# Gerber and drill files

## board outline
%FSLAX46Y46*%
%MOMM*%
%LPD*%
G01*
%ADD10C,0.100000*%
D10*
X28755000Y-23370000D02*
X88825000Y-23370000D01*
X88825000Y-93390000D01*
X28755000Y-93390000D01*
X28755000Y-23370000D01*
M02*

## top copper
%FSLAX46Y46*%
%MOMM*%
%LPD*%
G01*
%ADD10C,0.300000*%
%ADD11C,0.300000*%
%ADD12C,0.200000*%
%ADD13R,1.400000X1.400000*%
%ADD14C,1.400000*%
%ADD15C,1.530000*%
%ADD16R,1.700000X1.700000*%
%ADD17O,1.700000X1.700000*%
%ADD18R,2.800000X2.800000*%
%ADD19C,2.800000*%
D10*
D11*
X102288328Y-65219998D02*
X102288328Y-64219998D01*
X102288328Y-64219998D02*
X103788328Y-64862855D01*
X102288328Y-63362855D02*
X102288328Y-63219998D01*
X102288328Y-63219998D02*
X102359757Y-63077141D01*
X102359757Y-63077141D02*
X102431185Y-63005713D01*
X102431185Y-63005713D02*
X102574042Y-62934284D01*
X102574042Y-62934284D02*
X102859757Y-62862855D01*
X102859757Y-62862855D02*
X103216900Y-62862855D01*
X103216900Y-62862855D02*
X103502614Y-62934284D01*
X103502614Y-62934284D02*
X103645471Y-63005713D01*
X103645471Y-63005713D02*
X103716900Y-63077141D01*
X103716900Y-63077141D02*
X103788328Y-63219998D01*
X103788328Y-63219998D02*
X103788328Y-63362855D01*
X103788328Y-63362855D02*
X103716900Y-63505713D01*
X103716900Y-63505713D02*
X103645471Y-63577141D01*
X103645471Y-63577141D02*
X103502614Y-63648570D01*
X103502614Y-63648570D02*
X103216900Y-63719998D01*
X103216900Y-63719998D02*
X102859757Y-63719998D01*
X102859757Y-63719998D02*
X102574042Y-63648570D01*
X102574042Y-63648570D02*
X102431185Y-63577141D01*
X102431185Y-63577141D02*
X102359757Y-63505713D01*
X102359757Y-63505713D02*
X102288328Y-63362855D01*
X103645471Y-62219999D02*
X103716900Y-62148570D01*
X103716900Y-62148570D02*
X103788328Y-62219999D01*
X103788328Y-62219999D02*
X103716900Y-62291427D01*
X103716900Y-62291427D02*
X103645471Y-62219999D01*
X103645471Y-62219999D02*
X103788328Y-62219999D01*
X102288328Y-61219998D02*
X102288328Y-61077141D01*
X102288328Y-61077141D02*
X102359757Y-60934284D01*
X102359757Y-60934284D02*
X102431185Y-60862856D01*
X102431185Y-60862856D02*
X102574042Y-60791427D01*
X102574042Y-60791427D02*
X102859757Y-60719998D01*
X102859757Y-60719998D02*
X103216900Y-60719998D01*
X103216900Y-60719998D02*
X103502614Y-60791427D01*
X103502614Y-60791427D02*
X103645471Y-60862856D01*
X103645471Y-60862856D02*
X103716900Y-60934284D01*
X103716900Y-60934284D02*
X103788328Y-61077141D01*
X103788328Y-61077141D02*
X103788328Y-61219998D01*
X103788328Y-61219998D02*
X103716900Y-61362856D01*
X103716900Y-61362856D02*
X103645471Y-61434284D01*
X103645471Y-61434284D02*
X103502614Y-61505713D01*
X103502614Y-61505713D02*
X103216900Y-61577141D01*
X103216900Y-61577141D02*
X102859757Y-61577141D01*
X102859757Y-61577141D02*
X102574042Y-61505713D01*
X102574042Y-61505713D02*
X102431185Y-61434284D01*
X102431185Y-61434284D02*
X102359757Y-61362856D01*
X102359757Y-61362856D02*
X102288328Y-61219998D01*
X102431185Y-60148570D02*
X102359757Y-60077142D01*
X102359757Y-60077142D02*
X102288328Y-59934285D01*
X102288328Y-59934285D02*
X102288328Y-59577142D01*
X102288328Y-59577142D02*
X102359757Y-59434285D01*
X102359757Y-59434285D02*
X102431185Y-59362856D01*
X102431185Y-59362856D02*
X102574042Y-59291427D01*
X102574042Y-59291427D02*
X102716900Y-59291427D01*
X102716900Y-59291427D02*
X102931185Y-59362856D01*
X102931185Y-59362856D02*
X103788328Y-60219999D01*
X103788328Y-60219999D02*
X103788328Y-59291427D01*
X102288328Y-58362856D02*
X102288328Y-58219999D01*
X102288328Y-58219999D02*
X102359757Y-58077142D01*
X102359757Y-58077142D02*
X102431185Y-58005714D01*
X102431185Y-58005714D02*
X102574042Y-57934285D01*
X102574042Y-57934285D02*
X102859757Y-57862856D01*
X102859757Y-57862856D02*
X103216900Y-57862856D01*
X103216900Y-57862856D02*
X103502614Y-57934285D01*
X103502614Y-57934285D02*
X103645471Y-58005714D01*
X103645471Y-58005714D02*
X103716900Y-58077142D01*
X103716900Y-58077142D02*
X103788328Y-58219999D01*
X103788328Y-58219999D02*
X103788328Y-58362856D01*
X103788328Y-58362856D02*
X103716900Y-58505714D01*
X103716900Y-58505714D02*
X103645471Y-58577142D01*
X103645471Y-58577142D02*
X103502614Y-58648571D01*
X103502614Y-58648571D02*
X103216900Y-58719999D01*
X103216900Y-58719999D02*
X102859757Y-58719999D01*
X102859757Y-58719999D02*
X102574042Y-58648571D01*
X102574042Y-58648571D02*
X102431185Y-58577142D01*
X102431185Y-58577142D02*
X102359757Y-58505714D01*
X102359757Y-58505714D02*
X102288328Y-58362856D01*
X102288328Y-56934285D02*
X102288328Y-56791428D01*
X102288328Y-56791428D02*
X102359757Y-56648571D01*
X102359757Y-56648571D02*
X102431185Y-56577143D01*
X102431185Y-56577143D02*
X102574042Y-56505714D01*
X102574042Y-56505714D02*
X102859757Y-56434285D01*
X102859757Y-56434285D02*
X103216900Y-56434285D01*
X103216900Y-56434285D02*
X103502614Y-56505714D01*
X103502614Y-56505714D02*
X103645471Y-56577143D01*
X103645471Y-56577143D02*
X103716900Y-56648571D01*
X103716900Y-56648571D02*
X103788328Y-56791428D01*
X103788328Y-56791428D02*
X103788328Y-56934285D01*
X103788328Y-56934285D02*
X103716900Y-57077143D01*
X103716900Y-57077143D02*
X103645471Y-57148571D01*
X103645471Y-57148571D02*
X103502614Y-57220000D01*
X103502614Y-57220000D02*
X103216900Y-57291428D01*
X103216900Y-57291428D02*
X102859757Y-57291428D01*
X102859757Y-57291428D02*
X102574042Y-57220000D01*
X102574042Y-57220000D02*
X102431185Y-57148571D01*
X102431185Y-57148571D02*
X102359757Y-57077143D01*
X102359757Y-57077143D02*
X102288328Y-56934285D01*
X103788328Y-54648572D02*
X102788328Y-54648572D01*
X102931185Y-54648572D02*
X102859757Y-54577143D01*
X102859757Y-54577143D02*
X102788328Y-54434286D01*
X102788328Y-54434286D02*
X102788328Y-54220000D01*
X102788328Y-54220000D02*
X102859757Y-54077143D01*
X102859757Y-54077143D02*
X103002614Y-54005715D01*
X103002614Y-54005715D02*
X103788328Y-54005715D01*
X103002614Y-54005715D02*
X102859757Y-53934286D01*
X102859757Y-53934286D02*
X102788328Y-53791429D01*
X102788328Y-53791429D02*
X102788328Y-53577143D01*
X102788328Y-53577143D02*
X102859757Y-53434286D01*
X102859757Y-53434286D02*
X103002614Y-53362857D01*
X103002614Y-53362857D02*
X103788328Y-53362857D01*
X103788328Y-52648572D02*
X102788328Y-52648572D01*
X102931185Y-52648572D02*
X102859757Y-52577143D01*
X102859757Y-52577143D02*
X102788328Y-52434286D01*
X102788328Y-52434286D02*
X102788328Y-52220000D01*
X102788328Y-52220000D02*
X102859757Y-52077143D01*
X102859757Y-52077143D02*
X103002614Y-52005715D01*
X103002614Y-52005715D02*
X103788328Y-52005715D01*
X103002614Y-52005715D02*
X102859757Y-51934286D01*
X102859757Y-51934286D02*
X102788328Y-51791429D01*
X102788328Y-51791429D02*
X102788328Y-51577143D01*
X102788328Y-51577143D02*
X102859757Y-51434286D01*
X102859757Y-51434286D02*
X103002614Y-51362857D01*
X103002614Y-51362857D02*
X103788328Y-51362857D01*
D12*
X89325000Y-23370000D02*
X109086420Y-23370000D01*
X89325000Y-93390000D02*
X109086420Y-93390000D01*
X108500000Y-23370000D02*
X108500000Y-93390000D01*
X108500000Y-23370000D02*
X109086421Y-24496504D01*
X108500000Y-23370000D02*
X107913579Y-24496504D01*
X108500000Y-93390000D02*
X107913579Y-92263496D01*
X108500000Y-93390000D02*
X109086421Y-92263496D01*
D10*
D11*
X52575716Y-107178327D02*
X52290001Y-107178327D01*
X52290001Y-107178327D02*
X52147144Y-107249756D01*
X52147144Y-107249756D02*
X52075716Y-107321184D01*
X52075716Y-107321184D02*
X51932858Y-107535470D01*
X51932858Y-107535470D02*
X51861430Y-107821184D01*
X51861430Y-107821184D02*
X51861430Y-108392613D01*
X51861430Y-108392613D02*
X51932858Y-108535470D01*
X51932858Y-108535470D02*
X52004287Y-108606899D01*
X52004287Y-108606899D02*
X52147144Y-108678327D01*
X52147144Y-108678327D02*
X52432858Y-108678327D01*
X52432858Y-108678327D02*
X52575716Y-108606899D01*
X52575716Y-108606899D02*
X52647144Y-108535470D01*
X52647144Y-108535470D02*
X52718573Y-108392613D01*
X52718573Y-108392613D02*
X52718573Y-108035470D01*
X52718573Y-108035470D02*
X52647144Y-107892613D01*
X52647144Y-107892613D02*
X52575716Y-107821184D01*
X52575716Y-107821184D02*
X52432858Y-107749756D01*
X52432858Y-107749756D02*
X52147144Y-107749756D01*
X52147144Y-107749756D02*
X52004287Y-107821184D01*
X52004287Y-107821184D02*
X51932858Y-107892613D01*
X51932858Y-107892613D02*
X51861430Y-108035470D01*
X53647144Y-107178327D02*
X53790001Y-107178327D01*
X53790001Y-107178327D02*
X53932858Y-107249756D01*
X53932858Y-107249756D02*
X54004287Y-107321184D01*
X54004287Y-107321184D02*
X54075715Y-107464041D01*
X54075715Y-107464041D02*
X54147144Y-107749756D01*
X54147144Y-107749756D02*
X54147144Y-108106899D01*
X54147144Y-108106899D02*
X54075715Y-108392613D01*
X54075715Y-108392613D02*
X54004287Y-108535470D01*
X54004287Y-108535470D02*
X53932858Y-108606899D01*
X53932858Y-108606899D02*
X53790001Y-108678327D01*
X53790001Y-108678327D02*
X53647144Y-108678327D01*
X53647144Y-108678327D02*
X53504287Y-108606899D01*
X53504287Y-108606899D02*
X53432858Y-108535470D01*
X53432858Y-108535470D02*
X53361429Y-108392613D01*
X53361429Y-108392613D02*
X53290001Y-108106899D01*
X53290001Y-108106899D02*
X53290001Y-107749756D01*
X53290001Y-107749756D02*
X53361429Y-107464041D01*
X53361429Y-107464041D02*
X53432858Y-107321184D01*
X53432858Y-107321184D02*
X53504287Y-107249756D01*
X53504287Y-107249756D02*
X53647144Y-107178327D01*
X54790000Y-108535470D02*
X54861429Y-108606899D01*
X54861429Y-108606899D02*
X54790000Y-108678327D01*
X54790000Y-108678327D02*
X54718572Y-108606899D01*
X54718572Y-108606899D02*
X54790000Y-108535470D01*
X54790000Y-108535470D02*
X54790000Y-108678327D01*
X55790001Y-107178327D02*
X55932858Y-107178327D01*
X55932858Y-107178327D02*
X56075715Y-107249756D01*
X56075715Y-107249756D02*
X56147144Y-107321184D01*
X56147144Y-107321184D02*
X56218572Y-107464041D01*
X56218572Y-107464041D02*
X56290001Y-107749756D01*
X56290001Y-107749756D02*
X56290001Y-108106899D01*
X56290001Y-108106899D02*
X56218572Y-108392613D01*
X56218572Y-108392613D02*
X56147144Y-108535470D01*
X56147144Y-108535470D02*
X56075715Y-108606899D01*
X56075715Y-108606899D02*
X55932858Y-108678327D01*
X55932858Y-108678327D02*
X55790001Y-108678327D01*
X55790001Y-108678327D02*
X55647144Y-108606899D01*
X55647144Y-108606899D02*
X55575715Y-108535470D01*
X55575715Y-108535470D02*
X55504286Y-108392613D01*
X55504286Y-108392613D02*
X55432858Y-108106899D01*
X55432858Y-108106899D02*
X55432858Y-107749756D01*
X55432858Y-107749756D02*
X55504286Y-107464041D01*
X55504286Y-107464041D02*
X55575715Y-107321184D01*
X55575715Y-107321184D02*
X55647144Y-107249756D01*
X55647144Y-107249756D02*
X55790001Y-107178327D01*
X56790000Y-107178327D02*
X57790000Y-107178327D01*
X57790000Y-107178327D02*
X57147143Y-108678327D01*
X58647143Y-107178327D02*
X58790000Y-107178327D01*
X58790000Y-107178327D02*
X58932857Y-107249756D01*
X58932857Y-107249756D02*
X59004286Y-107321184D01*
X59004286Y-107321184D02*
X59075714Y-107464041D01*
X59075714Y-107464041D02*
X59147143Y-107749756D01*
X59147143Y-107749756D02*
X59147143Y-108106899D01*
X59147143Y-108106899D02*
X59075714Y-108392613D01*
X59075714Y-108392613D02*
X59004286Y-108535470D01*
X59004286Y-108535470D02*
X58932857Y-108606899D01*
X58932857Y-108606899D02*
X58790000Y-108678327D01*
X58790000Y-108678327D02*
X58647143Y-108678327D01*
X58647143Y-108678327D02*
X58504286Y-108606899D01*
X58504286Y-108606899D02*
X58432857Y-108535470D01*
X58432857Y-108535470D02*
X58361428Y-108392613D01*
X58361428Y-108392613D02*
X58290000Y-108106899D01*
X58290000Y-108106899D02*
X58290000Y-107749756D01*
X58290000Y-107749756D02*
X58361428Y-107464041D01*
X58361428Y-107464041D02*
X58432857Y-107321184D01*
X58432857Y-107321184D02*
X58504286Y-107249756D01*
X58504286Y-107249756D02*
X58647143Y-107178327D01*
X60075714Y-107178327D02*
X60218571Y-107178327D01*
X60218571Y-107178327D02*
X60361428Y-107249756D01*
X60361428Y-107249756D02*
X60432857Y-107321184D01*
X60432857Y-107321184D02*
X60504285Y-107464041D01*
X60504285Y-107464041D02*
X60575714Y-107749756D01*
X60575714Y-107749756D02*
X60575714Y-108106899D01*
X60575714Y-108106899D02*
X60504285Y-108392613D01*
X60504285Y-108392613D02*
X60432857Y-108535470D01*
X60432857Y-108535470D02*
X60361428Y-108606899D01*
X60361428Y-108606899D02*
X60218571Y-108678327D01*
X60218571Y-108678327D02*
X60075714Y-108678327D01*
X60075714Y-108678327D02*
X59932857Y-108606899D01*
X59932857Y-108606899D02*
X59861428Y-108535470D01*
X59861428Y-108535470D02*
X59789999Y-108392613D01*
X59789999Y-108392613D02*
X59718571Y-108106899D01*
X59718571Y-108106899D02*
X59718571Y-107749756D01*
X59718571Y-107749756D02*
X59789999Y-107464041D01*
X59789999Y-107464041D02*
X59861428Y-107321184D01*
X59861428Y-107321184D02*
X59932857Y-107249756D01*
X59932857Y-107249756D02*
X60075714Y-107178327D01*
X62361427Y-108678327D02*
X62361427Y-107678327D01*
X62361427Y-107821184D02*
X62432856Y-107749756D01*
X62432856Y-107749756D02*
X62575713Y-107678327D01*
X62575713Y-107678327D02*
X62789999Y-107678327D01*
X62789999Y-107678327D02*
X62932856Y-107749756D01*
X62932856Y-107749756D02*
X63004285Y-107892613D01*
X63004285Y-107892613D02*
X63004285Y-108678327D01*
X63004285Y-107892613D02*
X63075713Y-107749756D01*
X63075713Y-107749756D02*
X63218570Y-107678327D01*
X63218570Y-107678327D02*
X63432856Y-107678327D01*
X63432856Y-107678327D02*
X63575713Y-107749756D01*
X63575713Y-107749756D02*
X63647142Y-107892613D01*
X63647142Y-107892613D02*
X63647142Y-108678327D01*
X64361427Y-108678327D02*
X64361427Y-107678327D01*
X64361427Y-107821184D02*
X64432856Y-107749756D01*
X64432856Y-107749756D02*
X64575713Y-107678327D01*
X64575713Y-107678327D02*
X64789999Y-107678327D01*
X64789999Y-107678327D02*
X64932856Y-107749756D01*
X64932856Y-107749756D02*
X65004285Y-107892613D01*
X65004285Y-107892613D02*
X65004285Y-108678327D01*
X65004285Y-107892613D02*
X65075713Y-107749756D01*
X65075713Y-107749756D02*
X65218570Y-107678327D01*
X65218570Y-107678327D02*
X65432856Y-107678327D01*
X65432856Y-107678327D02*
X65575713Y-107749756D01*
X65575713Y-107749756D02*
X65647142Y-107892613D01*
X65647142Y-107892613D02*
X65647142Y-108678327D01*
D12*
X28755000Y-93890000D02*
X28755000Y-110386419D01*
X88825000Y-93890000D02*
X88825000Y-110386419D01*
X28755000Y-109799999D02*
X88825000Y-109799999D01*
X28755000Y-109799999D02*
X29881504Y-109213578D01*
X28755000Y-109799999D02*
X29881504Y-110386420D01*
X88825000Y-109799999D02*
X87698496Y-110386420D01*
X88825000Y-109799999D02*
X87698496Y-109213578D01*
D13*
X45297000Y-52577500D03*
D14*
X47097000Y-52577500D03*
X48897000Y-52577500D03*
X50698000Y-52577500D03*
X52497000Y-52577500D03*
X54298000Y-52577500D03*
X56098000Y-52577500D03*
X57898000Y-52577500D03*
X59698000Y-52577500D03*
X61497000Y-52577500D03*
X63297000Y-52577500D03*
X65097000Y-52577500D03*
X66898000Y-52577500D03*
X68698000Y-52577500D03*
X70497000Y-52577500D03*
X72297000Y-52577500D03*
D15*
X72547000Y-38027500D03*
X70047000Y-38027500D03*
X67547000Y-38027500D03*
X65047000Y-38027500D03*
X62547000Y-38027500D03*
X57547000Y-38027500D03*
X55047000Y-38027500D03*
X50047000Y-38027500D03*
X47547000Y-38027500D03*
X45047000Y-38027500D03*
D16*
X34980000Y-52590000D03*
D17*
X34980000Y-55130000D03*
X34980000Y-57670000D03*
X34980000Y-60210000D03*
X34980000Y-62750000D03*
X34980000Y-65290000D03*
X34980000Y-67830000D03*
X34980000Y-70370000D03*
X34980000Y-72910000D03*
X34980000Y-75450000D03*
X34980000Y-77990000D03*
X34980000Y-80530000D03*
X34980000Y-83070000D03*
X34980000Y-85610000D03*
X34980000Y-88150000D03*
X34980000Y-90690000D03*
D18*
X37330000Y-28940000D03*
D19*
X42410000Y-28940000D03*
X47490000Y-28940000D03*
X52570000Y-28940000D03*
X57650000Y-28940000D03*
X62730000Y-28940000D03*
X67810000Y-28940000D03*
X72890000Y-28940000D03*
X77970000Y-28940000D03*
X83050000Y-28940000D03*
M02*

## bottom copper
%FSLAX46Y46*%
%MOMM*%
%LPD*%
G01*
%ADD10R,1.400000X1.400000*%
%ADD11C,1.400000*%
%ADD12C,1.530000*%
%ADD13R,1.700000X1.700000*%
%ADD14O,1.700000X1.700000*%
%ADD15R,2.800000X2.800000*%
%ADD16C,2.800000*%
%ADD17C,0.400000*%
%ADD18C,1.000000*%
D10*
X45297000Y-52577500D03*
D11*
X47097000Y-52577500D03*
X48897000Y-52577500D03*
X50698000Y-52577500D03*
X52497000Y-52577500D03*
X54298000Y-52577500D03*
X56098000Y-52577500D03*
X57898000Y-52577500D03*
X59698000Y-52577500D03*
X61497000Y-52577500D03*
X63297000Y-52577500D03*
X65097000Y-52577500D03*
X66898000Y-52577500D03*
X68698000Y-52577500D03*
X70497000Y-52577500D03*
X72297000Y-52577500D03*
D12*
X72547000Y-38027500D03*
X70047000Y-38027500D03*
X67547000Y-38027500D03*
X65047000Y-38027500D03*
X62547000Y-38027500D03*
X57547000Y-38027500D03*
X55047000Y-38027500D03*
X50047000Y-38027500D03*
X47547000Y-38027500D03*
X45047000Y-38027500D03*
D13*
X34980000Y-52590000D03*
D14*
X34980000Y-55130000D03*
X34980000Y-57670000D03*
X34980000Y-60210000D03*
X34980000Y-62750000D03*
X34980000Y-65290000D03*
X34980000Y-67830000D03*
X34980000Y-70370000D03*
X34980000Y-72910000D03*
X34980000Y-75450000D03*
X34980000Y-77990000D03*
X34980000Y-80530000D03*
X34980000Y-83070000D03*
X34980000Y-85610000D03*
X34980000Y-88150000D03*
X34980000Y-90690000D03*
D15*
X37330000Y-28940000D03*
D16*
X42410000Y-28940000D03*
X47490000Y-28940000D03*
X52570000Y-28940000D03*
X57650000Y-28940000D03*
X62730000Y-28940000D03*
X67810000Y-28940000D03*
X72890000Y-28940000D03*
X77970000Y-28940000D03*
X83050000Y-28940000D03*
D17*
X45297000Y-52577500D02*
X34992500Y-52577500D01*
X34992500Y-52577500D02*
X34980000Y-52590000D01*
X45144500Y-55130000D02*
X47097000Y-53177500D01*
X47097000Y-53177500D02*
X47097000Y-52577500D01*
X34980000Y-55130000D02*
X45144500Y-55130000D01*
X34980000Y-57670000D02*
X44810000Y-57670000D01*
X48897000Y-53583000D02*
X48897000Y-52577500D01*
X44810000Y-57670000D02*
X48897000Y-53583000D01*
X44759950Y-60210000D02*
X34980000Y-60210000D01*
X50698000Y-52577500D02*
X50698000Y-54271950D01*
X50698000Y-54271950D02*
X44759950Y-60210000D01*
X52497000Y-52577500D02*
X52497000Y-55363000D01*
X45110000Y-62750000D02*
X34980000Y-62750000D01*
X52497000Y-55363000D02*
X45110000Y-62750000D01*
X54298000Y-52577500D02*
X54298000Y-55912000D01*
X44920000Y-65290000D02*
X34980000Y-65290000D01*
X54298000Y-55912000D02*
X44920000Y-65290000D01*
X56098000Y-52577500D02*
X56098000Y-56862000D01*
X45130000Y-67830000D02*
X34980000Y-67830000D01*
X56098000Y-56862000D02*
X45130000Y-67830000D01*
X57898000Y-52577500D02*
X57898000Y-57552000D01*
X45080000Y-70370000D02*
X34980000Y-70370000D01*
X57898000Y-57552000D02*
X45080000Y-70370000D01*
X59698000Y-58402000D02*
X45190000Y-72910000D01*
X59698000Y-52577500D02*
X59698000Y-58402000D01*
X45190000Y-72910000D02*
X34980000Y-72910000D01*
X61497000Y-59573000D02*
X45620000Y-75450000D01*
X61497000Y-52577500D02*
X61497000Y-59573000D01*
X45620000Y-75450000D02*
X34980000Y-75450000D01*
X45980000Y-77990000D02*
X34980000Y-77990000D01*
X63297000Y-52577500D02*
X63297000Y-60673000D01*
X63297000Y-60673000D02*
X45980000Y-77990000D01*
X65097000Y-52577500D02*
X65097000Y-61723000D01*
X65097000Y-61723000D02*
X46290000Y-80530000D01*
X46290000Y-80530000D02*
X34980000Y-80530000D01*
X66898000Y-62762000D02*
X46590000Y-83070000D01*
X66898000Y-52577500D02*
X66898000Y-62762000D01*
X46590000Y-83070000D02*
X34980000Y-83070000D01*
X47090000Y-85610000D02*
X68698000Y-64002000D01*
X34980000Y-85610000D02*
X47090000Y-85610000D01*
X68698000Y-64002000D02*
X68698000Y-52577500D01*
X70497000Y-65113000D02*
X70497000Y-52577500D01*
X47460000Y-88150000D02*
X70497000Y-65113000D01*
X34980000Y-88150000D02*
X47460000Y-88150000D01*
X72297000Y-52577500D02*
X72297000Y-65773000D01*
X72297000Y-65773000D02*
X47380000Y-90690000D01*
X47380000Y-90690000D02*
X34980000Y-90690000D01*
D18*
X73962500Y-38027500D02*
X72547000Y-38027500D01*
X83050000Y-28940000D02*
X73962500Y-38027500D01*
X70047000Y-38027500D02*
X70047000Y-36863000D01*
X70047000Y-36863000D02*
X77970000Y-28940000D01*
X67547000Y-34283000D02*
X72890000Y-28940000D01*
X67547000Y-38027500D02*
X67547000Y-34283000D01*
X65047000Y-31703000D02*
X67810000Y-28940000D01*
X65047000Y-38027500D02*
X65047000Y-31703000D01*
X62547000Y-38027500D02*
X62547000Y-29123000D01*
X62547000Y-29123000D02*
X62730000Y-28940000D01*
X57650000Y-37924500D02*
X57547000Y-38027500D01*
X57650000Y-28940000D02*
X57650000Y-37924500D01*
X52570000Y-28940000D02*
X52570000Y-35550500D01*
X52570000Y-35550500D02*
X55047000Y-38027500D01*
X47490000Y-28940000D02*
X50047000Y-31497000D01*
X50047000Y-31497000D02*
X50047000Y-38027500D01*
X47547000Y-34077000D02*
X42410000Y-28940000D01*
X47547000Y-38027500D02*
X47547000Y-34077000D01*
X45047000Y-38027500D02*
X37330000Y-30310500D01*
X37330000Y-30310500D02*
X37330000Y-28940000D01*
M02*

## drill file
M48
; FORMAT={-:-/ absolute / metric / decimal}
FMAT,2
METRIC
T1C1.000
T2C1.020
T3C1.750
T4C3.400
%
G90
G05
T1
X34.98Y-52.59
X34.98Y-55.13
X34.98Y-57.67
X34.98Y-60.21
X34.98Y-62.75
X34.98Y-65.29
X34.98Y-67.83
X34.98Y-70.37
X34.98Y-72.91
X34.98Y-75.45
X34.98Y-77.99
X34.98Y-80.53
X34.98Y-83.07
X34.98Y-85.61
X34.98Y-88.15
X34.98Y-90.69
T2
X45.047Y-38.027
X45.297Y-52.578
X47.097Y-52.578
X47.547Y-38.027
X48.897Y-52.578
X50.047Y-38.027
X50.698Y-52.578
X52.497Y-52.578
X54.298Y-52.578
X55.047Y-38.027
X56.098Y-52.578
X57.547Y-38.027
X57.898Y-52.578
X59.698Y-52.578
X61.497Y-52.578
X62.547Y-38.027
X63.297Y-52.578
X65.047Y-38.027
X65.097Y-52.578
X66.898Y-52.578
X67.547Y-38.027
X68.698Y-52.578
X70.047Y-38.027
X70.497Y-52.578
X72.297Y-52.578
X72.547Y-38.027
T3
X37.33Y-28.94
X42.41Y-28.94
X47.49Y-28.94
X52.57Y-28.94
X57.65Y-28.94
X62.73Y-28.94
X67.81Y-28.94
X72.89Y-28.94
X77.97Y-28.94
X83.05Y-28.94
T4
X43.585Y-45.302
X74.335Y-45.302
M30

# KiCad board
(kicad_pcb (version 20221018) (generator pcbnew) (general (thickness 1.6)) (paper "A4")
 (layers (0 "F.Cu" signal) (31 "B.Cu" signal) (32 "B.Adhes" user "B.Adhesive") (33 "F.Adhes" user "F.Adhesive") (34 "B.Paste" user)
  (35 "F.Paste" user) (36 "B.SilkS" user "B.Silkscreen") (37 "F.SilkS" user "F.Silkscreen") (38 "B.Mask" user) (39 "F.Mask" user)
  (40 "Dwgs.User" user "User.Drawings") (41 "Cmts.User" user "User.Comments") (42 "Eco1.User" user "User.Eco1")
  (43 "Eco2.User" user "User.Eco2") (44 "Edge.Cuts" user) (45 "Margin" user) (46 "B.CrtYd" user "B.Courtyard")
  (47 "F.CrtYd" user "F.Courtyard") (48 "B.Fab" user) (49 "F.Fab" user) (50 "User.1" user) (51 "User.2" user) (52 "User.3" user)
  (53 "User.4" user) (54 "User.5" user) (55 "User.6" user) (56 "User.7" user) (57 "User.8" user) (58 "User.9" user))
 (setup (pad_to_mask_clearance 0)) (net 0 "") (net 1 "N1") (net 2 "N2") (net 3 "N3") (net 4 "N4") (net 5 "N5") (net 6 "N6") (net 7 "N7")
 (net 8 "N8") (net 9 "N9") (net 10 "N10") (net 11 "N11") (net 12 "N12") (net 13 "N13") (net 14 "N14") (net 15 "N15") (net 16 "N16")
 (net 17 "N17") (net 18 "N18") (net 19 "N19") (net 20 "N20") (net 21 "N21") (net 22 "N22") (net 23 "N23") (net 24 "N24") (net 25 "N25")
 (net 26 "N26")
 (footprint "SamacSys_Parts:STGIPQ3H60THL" (layer "F.Cu") (at 45.297 52.5775)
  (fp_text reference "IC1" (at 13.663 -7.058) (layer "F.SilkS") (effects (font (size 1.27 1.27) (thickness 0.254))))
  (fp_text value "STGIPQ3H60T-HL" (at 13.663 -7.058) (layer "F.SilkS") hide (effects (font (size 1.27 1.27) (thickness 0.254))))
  (pad "" np_thru_hole circle (at -1.712 -7.275) (size 3.4 3.4) (drill 3.4) (layers "*.Cu" "*.Mask"))
  (pad "" np_thru_hole circle (at 29.038 -7.275) (size 3.4 3.4) (drill 3.4) (layers "*.Cu" "*.Mask"))
  (pad "1" thru_hole rect (at 0 0) (size 1.4 1.4) (drill 1.02) (layers "*.Cu" "*.Mask") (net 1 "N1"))
  (pad "2" thru_hole circle (at 1.8 0) (size 1.4 1.4) (drill 1.02) (layers "*.Cu" "*.Mask") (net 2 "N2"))
  (pad "3" thru_hole circle (at 3.6 0) (size 1.4 1.4) (drill 1.02) (layers "*.Cu" "*.Mask") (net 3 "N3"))
  (pad "4" thru_hole circle (at 5.401 0) (size 1.4 1.4) (drill 1.02) (layers "*.Cu" "*.Mask") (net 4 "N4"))
  (pad "5" thru_hole circle (at 7.2 0) (size 1.4 1.4) (drill 1.02) (layers "*.Cu" "*.Mask") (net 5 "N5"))
  (pad "6" thru_hole circle (at 9.001 0) (size 1.4 1.4) (drill 1.02) (layers "*.Cu" "*.Mask") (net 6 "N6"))
  (pad "7" thru_hole circle (at 10.801 0) (size 1.4 1.4) (drill 1.02) (layers "*.Cu" "*.Mask") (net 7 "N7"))
  (pad "8" thru_hole circle (at 12.601 0) (size 1.4 1.4) (drill 1.02) (layers "*.Cu" "*.Mask") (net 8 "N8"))
  (pad "9" thru_hole circle (at 14.401 0) (size 1.4 1.4) (drill 1.02) (layers "*.Cu" "*.Mask") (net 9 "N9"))
  (pad "10" thru_hole circle (at 16.2 0) (size 1.4 1.4) (drill 1.02) (layers "*.Cu" "*.Mask") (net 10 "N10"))
  (pad "11" thru_hole circle (at 18 0) (size 1.4 1.4) (drill 1.02) (layers "*.Cu" "*.Mask") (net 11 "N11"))
  (pad "12" thru_hole circle (at 19.8 0) (size 1.4 1.4) (drill 1.02) (layers "*.Cu" "*.Mask") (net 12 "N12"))
  (pad "13" thru_hole circle (at 21.601 0) (size 1.4 1.4) (drill 1.02) (layers "*.Cu" "*.Mask") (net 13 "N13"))
  (pad "14" thru_hole circle (at 23.401 0) (size 1.4 1.4) (drill 1.02) (layers "*.Cu" "*.Mask") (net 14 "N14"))
  (pad "15" thru_hole circle (at 25.2 0) (size 1.4 1.4) (drill 1.02) (layers "*.Cu" "*.Mask") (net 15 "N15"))
  (pad "16" thru_hole circle (at 27 0) (size 1.4 1.4) (drill 1.02) (layers "*.Cu" "*.Mask") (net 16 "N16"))
  (pad "17" thru_hole circle (at 27.25 -14.55) (size 1.53 1.53) (drill 1.02) (layers "*.Cu" "*.Mask") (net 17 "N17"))
  (pad "18" thru_hole circle (at 24.75 -14.55) (size 1.53 1.53) (drill 1.02) (layers "*.Cu" "*.Mask") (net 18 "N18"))
  (pad "19" thru_hole circle (at 22.25 -14.55) (size 1.53 1.53) (drill 1.02) (layers "*.Cu" "*.Mask") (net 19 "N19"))
  (pad "20" thru_hole circle (at 19.75 -14.55) (size 1.53 1.53) (drill 1.02) (layers "*.Cu" "*.Mask") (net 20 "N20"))
  (pad "21" thru_hole circle (at 17.25 -14.55) (size 1.53 1.53) (drill 1.02) (layers "*.Cu" "*.Mask") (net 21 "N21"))
  (pad "22" thru_hole circle (at 12.25 -14.55) (size 1.53 1.53) (drill 1.02) (layers "*.Cu" "*.Mask") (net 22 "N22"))
  (pad "23" thru_hole circle (at 9.75 -14.55) (size 1.53 1.53) (drill 1.02) (layers "*.Cu" "*.Mask") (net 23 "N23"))
  (pad "24" thru_hole circle (at 4.75 -14.55) (size 1.53 1.53) (drill 1.02) (layers "*.Cu" "*.Mask") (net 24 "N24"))
  (pad "25" thru_hole circle (at 2.25 -14.55) (size 1.53 1.53) (drill 1.02) (layers "*.Cu" "*.Mask") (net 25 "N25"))
  (pad "26" thru_hole circle (at -0.25 -14.55) (size 1.53 1.53) (drill 1.02) (layers "*.Cu" "*.Mask") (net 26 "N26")))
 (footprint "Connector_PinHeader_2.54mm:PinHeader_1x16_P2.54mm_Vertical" (layer "F.Cu") (at 34.98 52.59)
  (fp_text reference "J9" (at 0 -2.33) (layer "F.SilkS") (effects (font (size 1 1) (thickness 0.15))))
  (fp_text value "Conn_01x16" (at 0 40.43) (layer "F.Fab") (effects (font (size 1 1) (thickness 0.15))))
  (pad "1" thru_hole rect (at 0 0) (size 1.7 1.7) (drill 1) (layers "*.Cu" "*.Mask") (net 1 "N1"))
  (pad "2" thru_hole oval (at 0 2.54) (size 1.7 1.7) (drill 1) (layers "*.Cu" "*.Mask") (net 2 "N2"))
  (pad "3" thru_hole oval (at 0 5.08) (size 1.7 1.7) (drill 1) (layers "*.Cu" "*.Mask") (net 3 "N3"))
  (pad "4" thru_hole oval (at 0 7.62) (size 1.7 1.7) (drill 1) (layers "*.Cu" "*.Mask") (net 4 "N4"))
  (pad "5" thru_hole oval (at 0 10.16) (size 1.7 1.7) (drill 1) (layers "*.Cu" "*.Mask") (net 5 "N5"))
  (pad "6" thru_hole oval (at 0 12.7) (size 1.7 1.7) (drill 1) (layers "*.Cu" "*.Mask") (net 6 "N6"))
  (pad "7" thru_hole oval (at 0 15.24) (size 1.7 1.7) (drill 1) (layers "*.Cu" "*.Mask") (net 7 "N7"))
  (pad "8" thru_hole oval (at 0 17.78) (size 1.7 1.7) (drill 1) (layers "*.Cu" "*.Mask") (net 8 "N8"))
  (pad "9" thru_hole oval (at 0 20.32) (size 1.7 1.7) (drill 1) (layers "*.Cu" "*.Mask") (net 9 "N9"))
  (pad "10" thru_hole oval (at 0 22.86) (size 1.7 1.7) (drill 1) (layers "*.Cu" "*.Mask") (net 10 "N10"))
  (pad "11" thru_hole oval (at 0 25.4) (size 1.7 1.7) (drill 1) (layers "*.Cu" "*.Mask") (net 11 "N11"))
  (pad "12" thru_hole oval (at 0 27.94) (size 1.7 1.7) (drill 1) (layers "*.Cu" "*.Mask") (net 12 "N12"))
  (pad "13" thru_hole oval (at 0 30.48) (size 1.7 1.7) (drill 1) (layers "*.Cu" "*.Mask") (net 13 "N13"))
  (pad "14" thru_hole oval (at 0 33.02) (size 1.7 1.7) (drill 1) (layers "*.Cu" "*.Mask") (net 14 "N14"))
  (pad "15" thru_hole oval (at 0 35.56) (size 1.7 1.7) (drill 1) (layers "*.Cu" "*.Mask") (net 15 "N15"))
  (pad "16" thru_hole oval (at 0 38.1) (size 1.7 1.7) (drill 1) (layers "*.Cu" "*.Mask") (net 16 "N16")))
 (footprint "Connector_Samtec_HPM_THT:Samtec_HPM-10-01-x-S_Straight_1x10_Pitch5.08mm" (layer "F.Cu") (at 37.33 28.94 90)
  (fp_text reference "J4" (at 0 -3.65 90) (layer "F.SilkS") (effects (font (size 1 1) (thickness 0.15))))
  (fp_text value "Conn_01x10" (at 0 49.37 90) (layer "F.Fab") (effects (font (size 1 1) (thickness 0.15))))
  (pad "1" thru_hole rect (at 0 0 90) (size 2.8 2.8) (drill 1.75) (layers "*.Cu" "*.Mask") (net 26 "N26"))
  (pad "2" thru_hole circle (at 0 5.08 90) (size 2.8 2.8) (drill 1.75) (layers "*.Cu" "*.Mask") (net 25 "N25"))
  (pad "3" thru_hole circle (at 0 10.16 90) (size 2.8 2.8) (drill 1.75) (layers "*.Cu" "*.Mask") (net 24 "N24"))
  (pad "4" thru_hole circle (at 0 15.24 90) (size 2.8 2.8) (drill 1.75) (layers "*.Cu" "*.Mask") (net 23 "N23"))
  (pad "5" thru_hole circle (at 0 20.32 90) (size 2.8 2.8) (drill 1.75) (layers "*.Cu" "*.Mask") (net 22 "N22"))
  (pad "6" thru_hole circle (at 0 25.4 90) (size 2.8 2.8) (drill 1.75) (layers "*.Cu" "*.Mask") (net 21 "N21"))
  (pad "7" thru_hole circle (at 0 30.48 90) (size 2.8 2.8) (drill 1.75) (layers "*.Cu" "*.Mask") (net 20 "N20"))
  (pad "8" thru_hole circle (at 0 35.56 90) (size 2.8 2.8) (drill 1.75) (layers "*.Cu" "*.Mask") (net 19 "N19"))
  (pad "9" thru_hole circle (at 0 40.64 90) (size 2.8 2.8) (drill 1.75) (layers "*.Cu" "*.Mask") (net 18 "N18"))
  (pad "10" thru_hole circle (at 0 45.72 90) (size 2.8 2.8) (drill 1.75) (layers "*.Cu" "*.Mask") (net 17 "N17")))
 (gr_rect (start 28.755 23.37) (end 88.825 93.39) (stroke (width 0.1) (type default)) (fill none) (layer "Edge.Cuts"))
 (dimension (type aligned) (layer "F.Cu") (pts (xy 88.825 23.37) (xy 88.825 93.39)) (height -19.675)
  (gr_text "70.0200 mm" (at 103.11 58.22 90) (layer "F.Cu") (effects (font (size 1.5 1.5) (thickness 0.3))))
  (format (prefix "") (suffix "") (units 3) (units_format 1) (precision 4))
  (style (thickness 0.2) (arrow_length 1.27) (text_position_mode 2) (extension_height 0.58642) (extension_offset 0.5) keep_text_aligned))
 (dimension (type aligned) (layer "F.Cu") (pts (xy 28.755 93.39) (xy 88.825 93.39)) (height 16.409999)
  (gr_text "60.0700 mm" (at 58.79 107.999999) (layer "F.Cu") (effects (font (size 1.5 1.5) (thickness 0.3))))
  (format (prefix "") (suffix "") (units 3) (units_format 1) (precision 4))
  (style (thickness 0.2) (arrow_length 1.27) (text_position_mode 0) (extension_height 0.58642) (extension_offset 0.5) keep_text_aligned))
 (segment (start 45.297 52.5775) (end 34.9925 52.5775) (width 0.4) (layer "B.Cu") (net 1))
 (segment (start 34.9925 52.5775) (end 34.98 52.59) (width 0.4) (layer "B.Cu") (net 1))
 (segment (start 45.1445 55.13) (end 47.097 53.1775) (width 0.4) (layer "B.Cu") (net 2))
 (segment (start 47.097 53.1775) (end 47.097 52.5775) (width 0.4) (layer "B.Cu") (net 2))
 (segment (start 34.98 55.13) (end 45.1445 55.13) (width 0.4) (layer "B.Cu") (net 2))
 (segment (start 34.98 57.67) (end 44.81 57.67) (width 0.4) (layer "B.Cu") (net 3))
 (segment (start 48.897 53.583) (end 48.897 52.5775) (width 0.4) (layer "B.Cu") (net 3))
 (segment (start 44.81 57.67) (end 48.897 53.583) (width 0.4) (layer "B.Cu") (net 3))
 (segment (start 44.75995 60.21) (end 34.98 60.21) (width 0.4) (layer "B.Cu") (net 4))
 (segment (start 50.698 52.5775) (end 50.698 54.27195) (width 0.4) (layer "B.Cu") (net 4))
 (segment (start 50.698 54.27195) (end 44.75995 60.21) (width 0.4) (layer "B.Cu") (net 4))
 (segment (start 52.497 52.5775) (end 52.497 55.363) (width 0.4) (layer "B.Cu") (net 5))
 (segment (start 45.11 62.75) (end 34.98 62.75) (width 0.4) (layer "B.Cu") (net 5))
 (segment (start 52.497 55.363) (end 45.11 62.75) (width 0.4) (layer "B.Cu") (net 5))
 (segment (start 54.298 52.5775) (end 54.298 55.912) (width 0.4) (layer "B.Cu") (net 6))
 (segment (start 44.92 65.29) (end 34.98 65.29) (width 0.4) (layer "B.Cu") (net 6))
 (segment (start 54.298 55.912) (end 44.92 65.29) (width 0.4) (layer "B.Cu") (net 6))
 (segment (start 56.098 52.5775) (end 56.098 56.862) (width 0.4) (layer "B.Cu") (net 7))
 (segment (start 45.13 67.83) (end 34.98 67.83) (width 0.4) (layer "B.Cu") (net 7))
 (segment (start 56.098 56.862) (end 45.13 67.83) (width 0.4) (layer "B.Cu") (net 7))
 (segment (start 57.898 52.5775) (end 57.898 57.552) (width 0.4) (layer "B.Cu") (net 8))
 (segment (start 45.08 70.37) (end 34.98 70.37) (width 0.4) (layer "B.Cu") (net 8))
 (segment (start 57.898 57.552) (end 45.08 70.37) (width 0.4) (layer "B.Cu") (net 8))
 (segment (start 59.698 58.402) (end 45.19 72.91) (width 0.4) (layer "B.Cu") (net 9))
 (segment (start 59.698 52.5775) (end 59.698 58.402) (width 0.4) (layer "B.Cu") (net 9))
 (segment (start 45.19 72.91) (end 34.98 72.91) (width 0.4) (layer "B.Cu") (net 9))
 (segment (start 61.497 59.573) (end 45.62 75.45) (width 0.4) (layer "B.Cu") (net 10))
 (segment (start 61.497 52.5775) (end 61.497 59.573) (width 0.4) (layer "B.Cu") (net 10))
 (segment (start 45.62 75.45) (end 34.98 75.45) (width 0.4) (layer "B.Cu") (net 10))
 (segment (start 45.98 77.99) (end 34.98 77.99) (width 0.4) (layer "B.Cu") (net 11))
 (segment (start 63.297 52.5775) (end 63.297 60.673) (width 0.4) (layer "B.Cu") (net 11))
 (segment (start 63.297 60.673) (end 45.98 77.99) (width 0.4) (layer "B.Cu") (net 11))
 (segment (start 65.097 52.5775) (end 65.097 61.723) (width 0.4) (layer "B.Cu") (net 12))
 (segment (start 65.097 61.723) (end 46.29 80.53) (width 0.4) (layer "B.Cu") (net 12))
 (segment (start 46.29 80.53) (end 34.98 80.53) (width 0.4) (layer "B.Cu") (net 12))
 (segment (start 66.898 62.762) (end 46.59 83.07) (width 0.4) (layer "B.Cu") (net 13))
 (segment (start 66.898 52.5775) (end 66.898 62.762) (width 0.4) (layer "B.Cu") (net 13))
 (segment (start 46.59 83.07) (end 34.98 83.07) (width 0.4) (layer "B.Cu") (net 13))
 (segment (start 47.09 85.61) (end 68.698 64.002) (width 0.4) (layer "B.Cu") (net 14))
 (segment (start 34.98 85.61) (end 47.09 85.61) (width 0.4) (layer "B.Cu") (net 14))
 (segment (start 68.698 64.002) (end 68.698 52.5775) (width 0.4) (layer "B.Cu") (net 14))
 (segment (start 70.497 65.113) (end 70.497 52.5775) (width 0.4) (layer "B.Cu") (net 15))
 (segment (start 47.46 88.15) (end 70.497 65.113) (width 0.4) (layer "B.Cu") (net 15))
 (segment (start 34.98 88.15) (end 47.46 88.15) (width 0.4) (layer "B.Cu") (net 15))
 (segment (start 72.297 52.5775) (end 72.297 65.773) (width 0.4) (layer "B.Cu") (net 16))
 (segment (start 72.297 65.773) (end 47.38 90.69) (width 0.4) (layer "B.Cu") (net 16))
 (segment (start 47.38 90.69) (end 34.98 90.69) (width 0.4) (layer "B.Cu") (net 16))
 (segment (start 73.9625 38.0275) (end 72.547 38.0275) (width 1) (layer "B.Cu") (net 17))
 (segment (start 83.05 28.94) (end 73.9625 38.0275) (width 1) (layer "B.Cu") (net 17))
 (segment (start 70.047 38.0275) (end 70.047 36.863) (width 1) (layer "B.Cu") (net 18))
 (segment (start 70.047 36.863) (end 77.97 28.94) (width 1) (layer "B.Cu") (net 18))
 (segment (start 67.547 34.283) (end 72.89 28.94) (width 1) (layer "B.Cu") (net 19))
 (segment (start 67.547 38.0275) (end 67.547 34.283) (width 1) (layer "B.Cu") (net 19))
 (segment (start 65.047 31.703) (end 67.81 28.94) (width 1) (layer "B.Cu") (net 20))
 (segment (start 65.047 38.0275) (end 65.047 31.703) (width 1) (layer "B.Cu") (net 20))
 (segment (start 62.547 38.0275) (end 62.547 29.123) (width 1) (layer "B.Cu") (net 21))
 (segment (start 62.547 29.123) (end 62.73 28.94) (width 1) (layer "B.Cu") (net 21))
 (segment (start 57.65 37.9245) (end 57.547 38.0275) (width 1) (layer "B.Cu") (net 22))
 (segment (start 57.65 28.94) (end 57.65 37.9245) (width 1) (layer "B.Cu") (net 22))
 (segment (start 52.57 28.94) (end 52.57 35.5505) (width 1) (layer "B.Cu") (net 23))
 (segment (start 52.57 35.5505) (end 55.047 38.0275) (width 1) (layer "B.Cu") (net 23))
 (segment (start 47.49 28.94) (end 50.047 31.497) (width 1) (layer "B.Cu") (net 24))
 (segment (start 50.047 31.497) (end 50.047 38.0275) (width 1) (layer "B.Cu") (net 24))
 (segment (start 47.547 34.077) (end 42.41 28.94) (width 1) (layer "B.Cu") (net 25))
 (segment (start 47.547 38.0275) (end 47.547 34.077) (width 1) (layer "B.Cu") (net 25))
 (segment (start 45.047 38.0275) (end 37.33 30.3105) (width 1) (layer "B.Cu") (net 26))
 (segment (start 37.33 30.3105) (end 37.33 28.94) (width 1) (layer "B.Cu") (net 26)))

